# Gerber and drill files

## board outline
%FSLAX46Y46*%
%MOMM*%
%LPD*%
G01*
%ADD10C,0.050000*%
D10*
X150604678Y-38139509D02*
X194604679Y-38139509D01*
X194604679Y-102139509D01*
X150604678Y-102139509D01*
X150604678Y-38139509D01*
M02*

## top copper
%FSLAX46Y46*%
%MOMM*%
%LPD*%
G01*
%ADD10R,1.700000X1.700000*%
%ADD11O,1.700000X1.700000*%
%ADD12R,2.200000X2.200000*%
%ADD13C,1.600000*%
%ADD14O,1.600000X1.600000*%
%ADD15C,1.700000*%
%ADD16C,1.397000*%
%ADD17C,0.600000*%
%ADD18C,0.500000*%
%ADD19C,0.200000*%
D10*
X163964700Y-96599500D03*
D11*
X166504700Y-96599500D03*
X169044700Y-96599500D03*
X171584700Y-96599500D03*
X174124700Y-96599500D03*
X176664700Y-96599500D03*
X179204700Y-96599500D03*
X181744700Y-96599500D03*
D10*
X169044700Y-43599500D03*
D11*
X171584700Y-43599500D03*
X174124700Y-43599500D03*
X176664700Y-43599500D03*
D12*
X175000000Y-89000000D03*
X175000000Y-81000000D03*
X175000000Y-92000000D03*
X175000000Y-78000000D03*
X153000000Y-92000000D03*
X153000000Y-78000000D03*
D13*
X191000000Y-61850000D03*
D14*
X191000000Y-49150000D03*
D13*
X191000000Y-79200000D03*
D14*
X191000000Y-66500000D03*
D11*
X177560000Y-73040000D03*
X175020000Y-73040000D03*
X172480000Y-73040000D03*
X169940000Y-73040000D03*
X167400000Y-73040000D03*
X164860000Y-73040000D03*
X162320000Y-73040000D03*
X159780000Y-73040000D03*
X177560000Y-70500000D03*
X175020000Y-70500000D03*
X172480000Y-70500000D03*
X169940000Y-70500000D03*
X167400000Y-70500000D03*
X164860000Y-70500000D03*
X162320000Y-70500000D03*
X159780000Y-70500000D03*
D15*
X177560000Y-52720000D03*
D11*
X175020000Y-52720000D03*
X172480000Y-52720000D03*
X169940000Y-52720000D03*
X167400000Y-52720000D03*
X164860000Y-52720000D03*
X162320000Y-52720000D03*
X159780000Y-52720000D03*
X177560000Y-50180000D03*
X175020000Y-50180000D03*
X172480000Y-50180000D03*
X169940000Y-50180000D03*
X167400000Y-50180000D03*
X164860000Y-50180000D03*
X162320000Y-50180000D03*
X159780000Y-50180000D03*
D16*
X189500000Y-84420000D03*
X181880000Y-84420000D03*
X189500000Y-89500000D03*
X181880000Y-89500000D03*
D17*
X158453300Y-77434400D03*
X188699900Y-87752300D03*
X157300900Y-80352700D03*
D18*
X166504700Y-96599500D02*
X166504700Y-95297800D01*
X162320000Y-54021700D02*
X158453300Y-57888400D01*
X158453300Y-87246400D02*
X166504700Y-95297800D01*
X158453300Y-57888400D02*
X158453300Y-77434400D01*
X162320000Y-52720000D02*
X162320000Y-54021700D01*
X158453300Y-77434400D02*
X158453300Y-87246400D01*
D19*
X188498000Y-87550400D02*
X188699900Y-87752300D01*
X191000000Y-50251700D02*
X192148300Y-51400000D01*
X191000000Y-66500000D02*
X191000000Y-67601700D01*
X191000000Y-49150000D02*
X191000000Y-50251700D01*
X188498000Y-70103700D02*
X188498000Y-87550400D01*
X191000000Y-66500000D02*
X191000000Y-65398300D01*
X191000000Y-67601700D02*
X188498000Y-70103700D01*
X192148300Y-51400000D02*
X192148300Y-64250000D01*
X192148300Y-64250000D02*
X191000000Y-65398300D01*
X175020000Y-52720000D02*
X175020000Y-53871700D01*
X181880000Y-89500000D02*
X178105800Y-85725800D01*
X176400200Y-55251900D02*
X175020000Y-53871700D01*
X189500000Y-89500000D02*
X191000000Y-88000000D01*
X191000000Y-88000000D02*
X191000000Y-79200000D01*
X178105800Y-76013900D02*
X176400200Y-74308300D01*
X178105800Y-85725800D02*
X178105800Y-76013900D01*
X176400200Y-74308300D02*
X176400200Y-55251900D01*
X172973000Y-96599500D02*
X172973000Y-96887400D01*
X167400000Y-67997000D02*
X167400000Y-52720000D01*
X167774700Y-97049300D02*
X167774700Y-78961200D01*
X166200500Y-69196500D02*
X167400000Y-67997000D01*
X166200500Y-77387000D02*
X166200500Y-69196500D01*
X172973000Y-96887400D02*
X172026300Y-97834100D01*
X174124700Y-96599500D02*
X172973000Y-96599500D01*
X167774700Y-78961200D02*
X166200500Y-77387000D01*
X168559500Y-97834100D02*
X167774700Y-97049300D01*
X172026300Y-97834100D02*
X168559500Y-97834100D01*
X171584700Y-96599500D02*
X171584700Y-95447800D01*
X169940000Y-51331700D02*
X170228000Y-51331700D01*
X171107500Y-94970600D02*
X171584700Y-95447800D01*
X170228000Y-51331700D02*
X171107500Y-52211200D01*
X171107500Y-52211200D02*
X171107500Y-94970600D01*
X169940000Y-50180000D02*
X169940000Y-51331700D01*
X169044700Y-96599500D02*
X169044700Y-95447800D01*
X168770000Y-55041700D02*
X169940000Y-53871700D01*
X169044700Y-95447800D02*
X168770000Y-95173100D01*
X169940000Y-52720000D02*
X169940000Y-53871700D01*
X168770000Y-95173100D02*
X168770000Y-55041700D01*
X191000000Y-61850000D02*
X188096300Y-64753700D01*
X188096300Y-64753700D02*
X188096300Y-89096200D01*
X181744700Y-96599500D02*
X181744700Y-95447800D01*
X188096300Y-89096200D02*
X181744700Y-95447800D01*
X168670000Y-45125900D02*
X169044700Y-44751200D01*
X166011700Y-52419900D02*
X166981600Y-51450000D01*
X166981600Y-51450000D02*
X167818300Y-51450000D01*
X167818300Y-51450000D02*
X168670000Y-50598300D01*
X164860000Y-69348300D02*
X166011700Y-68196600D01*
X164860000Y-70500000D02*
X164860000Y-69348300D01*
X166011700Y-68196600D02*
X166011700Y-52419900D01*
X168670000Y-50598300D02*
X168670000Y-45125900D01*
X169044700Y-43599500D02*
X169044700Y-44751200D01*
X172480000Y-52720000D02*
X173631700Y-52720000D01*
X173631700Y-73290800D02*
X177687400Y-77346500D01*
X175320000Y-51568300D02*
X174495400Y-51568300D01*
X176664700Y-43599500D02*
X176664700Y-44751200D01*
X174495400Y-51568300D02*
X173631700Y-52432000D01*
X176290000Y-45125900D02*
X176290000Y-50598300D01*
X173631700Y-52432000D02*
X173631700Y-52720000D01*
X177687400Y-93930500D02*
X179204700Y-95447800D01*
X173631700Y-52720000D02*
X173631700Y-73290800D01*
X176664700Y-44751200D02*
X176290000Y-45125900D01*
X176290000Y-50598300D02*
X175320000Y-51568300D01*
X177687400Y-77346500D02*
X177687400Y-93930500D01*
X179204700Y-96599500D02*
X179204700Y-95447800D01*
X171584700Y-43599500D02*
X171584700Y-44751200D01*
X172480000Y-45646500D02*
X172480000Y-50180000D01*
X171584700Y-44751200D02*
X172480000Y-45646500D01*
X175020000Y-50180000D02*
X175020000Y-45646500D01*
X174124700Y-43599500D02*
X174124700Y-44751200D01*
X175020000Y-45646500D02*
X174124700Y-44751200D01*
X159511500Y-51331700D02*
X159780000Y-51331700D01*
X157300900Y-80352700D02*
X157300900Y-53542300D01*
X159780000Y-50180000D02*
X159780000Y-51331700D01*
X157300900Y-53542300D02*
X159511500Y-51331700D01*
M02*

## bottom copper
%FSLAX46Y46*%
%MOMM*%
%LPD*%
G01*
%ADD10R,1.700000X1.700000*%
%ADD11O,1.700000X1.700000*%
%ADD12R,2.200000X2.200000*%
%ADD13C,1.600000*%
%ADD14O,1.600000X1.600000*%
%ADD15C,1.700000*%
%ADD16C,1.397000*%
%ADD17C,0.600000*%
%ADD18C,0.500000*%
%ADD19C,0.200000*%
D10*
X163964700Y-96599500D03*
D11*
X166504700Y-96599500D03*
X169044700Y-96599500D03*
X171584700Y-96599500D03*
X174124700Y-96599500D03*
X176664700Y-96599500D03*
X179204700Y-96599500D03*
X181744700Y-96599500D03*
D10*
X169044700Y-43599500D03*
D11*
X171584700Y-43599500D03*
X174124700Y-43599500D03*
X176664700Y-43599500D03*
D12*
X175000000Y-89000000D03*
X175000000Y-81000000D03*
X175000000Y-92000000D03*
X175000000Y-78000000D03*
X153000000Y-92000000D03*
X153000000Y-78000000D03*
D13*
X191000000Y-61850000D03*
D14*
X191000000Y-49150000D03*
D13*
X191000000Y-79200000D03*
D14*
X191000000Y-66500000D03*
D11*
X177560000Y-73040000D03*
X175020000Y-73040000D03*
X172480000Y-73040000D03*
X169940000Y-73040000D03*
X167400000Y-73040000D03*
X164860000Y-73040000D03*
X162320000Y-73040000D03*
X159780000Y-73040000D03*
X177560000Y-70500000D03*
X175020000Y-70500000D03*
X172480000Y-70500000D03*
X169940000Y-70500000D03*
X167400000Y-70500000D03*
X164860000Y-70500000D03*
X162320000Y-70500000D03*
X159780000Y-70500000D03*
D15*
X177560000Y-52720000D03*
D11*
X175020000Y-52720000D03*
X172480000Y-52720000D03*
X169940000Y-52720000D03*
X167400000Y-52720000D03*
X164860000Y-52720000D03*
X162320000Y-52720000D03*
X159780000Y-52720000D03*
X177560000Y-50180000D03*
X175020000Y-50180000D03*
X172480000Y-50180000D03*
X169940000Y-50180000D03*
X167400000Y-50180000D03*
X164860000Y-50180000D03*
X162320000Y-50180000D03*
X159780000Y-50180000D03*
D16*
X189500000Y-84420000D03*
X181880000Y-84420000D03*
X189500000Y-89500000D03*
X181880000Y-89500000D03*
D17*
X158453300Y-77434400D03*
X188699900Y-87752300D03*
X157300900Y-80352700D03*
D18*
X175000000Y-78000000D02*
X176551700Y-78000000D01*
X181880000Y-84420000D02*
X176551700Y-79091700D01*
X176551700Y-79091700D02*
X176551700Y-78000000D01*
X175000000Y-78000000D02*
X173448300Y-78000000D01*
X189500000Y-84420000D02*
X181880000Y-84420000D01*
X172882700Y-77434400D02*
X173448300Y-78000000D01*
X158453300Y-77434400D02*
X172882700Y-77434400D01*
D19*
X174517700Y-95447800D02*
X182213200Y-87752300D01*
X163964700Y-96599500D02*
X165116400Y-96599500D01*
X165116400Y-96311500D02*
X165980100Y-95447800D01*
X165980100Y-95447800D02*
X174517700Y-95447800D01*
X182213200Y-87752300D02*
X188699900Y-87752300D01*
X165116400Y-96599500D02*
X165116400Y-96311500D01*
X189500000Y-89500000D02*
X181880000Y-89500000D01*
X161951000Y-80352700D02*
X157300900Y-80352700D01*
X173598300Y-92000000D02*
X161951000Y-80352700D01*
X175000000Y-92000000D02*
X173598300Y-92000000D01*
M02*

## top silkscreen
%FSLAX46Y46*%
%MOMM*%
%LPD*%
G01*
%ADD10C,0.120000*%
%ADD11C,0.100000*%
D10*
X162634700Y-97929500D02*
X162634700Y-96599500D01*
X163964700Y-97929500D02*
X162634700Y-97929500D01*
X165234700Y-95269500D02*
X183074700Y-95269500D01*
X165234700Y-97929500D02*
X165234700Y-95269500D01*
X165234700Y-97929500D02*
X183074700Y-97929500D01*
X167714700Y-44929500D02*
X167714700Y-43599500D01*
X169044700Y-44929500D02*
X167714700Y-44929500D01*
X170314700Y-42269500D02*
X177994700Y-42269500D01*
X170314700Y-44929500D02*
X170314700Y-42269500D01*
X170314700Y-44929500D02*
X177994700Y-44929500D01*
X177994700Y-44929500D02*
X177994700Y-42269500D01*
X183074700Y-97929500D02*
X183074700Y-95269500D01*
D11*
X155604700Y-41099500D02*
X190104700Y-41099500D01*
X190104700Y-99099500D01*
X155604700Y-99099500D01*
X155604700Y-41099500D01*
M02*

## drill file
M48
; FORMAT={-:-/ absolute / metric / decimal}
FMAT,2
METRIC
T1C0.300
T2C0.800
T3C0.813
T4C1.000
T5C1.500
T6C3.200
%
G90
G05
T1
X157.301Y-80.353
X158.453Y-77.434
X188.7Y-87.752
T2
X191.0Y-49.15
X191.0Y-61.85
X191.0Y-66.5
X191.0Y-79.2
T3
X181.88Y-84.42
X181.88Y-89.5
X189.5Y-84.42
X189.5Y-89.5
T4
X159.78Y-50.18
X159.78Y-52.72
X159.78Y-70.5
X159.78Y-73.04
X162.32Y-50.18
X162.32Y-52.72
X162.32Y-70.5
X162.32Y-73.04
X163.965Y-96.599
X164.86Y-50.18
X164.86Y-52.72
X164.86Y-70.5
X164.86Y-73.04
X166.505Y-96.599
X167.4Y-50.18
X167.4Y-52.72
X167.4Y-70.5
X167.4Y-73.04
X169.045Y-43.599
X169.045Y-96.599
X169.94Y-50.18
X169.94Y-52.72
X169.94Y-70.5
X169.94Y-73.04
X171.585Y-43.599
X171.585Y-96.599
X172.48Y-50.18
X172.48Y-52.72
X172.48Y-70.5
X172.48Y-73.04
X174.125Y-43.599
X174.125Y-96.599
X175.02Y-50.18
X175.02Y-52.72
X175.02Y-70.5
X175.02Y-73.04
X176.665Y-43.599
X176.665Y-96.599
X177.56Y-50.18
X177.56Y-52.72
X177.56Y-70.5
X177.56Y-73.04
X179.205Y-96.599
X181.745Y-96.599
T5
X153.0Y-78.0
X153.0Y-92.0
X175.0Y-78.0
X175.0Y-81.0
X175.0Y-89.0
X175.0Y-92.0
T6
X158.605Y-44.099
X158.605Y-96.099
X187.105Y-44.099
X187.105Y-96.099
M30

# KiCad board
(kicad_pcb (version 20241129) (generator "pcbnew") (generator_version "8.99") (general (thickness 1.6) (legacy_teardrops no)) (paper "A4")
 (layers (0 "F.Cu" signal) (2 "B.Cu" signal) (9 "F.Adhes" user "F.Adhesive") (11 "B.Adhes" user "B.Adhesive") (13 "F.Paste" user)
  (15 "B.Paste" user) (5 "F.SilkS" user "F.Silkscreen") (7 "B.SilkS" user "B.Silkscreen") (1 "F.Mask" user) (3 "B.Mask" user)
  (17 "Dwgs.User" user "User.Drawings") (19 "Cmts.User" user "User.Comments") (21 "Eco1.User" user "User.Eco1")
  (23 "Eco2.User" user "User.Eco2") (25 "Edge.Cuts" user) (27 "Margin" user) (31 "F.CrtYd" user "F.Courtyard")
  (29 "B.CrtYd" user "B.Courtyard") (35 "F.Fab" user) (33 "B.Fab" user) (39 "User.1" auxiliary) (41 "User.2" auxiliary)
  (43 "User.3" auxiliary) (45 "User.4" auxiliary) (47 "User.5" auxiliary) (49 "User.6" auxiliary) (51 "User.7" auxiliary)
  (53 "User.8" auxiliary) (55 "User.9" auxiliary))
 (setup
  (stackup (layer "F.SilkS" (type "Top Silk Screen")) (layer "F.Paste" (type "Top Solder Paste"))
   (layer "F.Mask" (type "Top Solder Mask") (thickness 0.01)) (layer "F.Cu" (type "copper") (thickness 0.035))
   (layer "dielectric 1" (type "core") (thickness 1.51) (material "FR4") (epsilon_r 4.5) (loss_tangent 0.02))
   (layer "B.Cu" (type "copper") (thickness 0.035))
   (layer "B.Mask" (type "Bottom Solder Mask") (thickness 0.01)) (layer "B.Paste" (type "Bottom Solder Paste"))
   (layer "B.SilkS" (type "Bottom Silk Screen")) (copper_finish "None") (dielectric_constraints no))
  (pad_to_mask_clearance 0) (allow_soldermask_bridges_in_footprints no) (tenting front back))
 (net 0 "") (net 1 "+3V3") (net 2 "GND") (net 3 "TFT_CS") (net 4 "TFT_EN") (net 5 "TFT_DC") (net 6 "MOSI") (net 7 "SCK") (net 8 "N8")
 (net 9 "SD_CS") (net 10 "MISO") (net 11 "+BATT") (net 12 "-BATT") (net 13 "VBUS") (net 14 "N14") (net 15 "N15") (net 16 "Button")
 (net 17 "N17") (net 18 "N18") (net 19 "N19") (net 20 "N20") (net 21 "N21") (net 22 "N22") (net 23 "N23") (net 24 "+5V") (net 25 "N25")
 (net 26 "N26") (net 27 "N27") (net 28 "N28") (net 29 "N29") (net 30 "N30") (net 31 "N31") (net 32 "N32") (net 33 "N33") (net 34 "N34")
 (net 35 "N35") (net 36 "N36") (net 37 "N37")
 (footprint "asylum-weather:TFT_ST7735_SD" (layer "F.Cu") (at 172.6047 76.5995 90)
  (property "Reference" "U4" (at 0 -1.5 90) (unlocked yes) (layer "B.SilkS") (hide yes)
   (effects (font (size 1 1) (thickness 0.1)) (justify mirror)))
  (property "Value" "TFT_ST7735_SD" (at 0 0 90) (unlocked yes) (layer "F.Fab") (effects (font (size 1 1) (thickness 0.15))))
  (fp_line (start -21.33 -9.97) (end -20 -9.97) (stroke (width 0.12) (type solid)) (layer "F.SilkS"))
  (fp_line (start -21.33 -8.64) (end -21.33 -9.97) (stroke (width 0.12) (type solid)) (layer "F.SilkS"))
  (fp_line (start -18.67 -7.37) (end -18.67 10.47) (stroke (width 0.12) (type solid)) (layer "F.SilkS"))
  (fp_line (start -21.33 -7.37) (end -18.67 -7.37) (stroke (width 0.12) (type solid)) (layer "F.SilkS"))
  (fp_line (start -21.33 -7.37) (end -21.33 10.47) (stroke (width 0.12) (type solid)) (layer "F.SilkS"))
  (fp_line (start 31.67 -4.89) (end 33 -4.89) (stroke (width 0.12) (type solid)) (layer "F.SilkS"))
  (fp_line (start 31.67 -3.56) (end 31.67 -4.89) (stroke (width 0.12) (type solid)) (layer "F.SilkS"))
  (fp_line (start 34.33 -2.29) (end 34.33 5.39) (stroke (width 0.12) (type solid)) (layer "F.SilkS"))
  (fp_line (start 31.67 -2.29) (end 34.33 -2.29) (stroke (width 0.12) (type solid)) (layer "F.SilkS"))
  (fp_line (start 31.67 -2.29) (end 31.67 5.39) (stroke (width 0.12) (type solid)) (layer "F.SilkS"))
  (fp_line (start 31.67 5.39) (end 34.33 5.39) (stroke (width 0.12) (type solid)) (layer "F.SilkS"))
  (fp_line (start -21.33 10.47) (end -18.67 10.47) (stroke (width 0.12) (type solid)) (layer "F.SilkS"))
  (fp_rect (start -22.5 -17) (end 35.5 17.5) (stroke (width 0.1) (type default)) (fill no) (layer "F.SilkS"))
  (pad "" np_thru_hole circle (at -19.5 -14 90) (size 3.2 3.2) (drill 3.2) (layers "*.Cu" "*.Mask"))
  (pad "" np_thru_hole circle (at -19.5 14.5 90) (size 3.2 3.2) (drill 3.2) (layers "*.Cu" "*.Mask"))
  (pad "" np_thru_hole circle (at 32.5 -14 90) (size 3.2 3.2) (drill 3.2) (layers "*.Cu" "*.Mask"))
  (pad "" np_thru_hole circle (at 32.5 14.5 90) (size 3.2 3.2) (drill 3.2) (layers "*.Cu" "*.Mask"))
  (pad "1" thru_hole rect (at -20 -8.64 90) (size 1.7 1.7) (drill 1) (layers "*.Cu" "*.Mask") (remove_unused_layers no) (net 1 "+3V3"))
  (pad "2" thru_hole oval (at -20 -6.1 90) (size 1.7 1.7) (drill 1) (layers "*.Cu" "*.Mask") (remove_unused_layers no) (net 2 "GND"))
  (pad "3" thru_hole oval (at -20 -3.56 90) (size 1.7 1.7) (drill 1) (layers "*.Cu" "*.Mask") (remove_unused_layers no) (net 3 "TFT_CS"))
  (pad "4" thru_hole oval (at -20 -1.02 90) (size 1.7 1.7) (drill 1) (layers "*.Cu" "*.Mask") (remove_unused_layers no) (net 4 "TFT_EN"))
  (pad "5" thru_hole oval (at -20 1.52 90) (size 1.7 1.7) (drill 1) (layers "*.Cu" "*.Mask") (remove_unused_layers no) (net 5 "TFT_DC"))
  (pad "6" thru_hole oval (at -20 4.06 90) (size 1.7 1.7) (drill 1) (layers "*.Cu" "*.Mask") (remove_unused_layers no) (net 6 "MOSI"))
  (pad "7" thru_hole oval (at -20 6.6 90) (size 1.7 1.7) (drill 1) (layers "*.Cu" "*.Mask") (remove_unused_layers no) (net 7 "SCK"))
  (pad "8" thru_hole oval (at -20 9.14 90) (size 1.7 1.7) (drill 1) (layers "*.Cu" "*.Mask") (remove_unused_layers no) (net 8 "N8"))
  (pad "9" thru_hole rect (at 33 -3.56 90) (size 1.7 1.7) (drill 1) (layers "*.Cu" "*.Mask") (remove_unused_layers no) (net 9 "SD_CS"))
  (pad "10" thru_hole oval (at 33 -1.02 90) (size 1.7 1.7) (drill 1) (layers "*.Cu" "*.Mask") (remove_unused_layers no) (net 6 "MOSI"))
  (pad "11" thru_hole oval (at 33 1.52 90) (size 1.7 1.7) (drill 1) (layers "*.Cu" "*.Mask") (remove_unused_layers no) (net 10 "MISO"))
  (pad "12" thru_hole oval (at 33 4.06 90) (size 1.7 1.7) (drill 1) (layers "*.Cu" "*.Mask") (remove_unused_layers no) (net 7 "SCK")))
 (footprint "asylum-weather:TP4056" (layer "B.Cu") (at 164.5 85 -90)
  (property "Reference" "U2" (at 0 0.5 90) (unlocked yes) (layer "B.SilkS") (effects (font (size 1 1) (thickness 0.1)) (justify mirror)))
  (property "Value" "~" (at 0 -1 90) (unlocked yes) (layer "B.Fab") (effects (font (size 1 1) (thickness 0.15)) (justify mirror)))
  (pad "0" thru_hole rect (at 4 -10.5 180) (size 2.2 2.2) (drill 1.5) (layers "F&B.Cu" "*.Mask") (remove_unused_layers no) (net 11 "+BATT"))
  (pad "1" thru_hole rect (at -4 -10.5 180) (size 2.2 2.2) (drill 1.5) (layers "F&B.Cu" "*.Mask") (remove_unused_layers no) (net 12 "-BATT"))
  (pad "2" thru_hole rect (at 7 -10.5 180) (size 2.2 2.2) (drill 1.5) (layers "F&B.Cu" "*.Mask") (remove_unused_layers no) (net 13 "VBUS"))
  (pad "3" thru_hole rect (at -7 -10.5 180) (size 2.2 2.2) (drill 1.5) (layers "F&B.Cu" "*.Mask") (remove_unused_layers no) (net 2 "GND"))
  (pad "4" thru_hole rect (at 7 11.5 180) (size 2.2 2.2) (drill 1.5) (layers "F&B.Cu" "*.Mask") (remove_unused_layers no) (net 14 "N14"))
  (pad "5" thru_hole rect (at -7 11.5 180) (size 2.2 2.2) (drill 1.5) (layers "F&B.Cu" "*.Mask") (remove_unused_layers no) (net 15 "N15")))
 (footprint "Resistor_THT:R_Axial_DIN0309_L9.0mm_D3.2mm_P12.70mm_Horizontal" (layer "B.Cu") (at 191 61.85 90)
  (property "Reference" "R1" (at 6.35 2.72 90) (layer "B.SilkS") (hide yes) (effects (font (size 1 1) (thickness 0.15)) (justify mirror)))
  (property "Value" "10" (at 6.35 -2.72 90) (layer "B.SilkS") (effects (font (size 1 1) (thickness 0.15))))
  (pad "1" thru_hole circle (at 0 0 90) (size 1.6 1.6) (drill 0.8) (layers "F&B.Cu" "*.Mask") (remove_unused_layers no) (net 8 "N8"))
  (pad "2" thru_hole oval (at 12.7 0 90) (size 1.6 1.6) (drill 0.8) (layers "F&B.Cu" "*.Mask") (remove_unused_layers no) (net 1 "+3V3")))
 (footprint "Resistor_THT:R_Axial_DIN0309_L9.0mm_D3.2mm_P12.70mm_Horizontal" (layer "B.Cu") (at 191 79.2 90)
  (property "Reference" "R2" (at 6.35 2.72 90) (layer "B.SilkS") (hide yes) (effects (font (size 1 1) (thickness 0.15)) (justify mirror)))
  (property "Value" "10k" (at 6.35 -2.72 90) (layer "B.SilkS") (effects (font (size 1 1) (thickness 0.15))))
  (pad "1" thru_hole circle (at 0 0 90) (size 1.6 1.6) (drill 0.8) (layers "F&B.Cu" "*.Mask") (remove_unused_layers no) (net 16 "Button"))
  (pad "2" thru_hole oval (at 12.7 0 90) (size 1.6 1.6) (drill 0.8) (layers "F&B.Cu" "*.Mask") (remove_unused_layers no) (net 1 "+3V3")))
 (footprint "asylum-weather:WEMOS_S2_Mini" (layer "B.Cu") (at 170.06 61.61 90)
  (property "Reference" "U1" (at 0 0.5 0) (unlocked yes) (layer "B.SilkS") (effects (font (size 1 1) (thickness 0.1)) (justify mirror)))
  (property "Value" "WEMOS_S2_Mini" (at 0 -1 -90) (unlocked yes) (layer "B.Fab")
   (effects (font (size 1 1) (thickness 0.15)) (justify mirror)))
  (pad "1" thru_hole oval (at -11.43 7.5 90) (size 1.7 1.7) (drill 1) (layers "F&B.Cu" "*.Mask") (remove_unused_layers no) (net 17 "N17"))
  (pad "2" thru_hole oval (at -11.43 4.96 90) (size 1.7 1.7) (drill 1) (layers "F&B.Cu" "*.Mask") (remove_unused_layers no) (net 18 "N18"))
  (pad "3" thru_hole oval (at -11.43 2.42 90) (size 1.7 1.7) (drill 1) (layers "F&B.Cu" "*.Mask") (remove_unused_layers no) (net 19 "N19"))
  (pad "4" thru_hole oval (at -11.43 -0.12 90) (size 1.7 1.7) (drill 1) (layers "F&B.Cu" "*.Mask") (remove_unused_layers no) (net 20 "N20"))
  (pad "5" thru_hole oval (at -11.43 -2.66 90) (size 1.7 1.7) (drill 1) (layers "F&B.Cu" "*.Mask") (remove_unused_layers no) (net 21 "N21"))
  (pad "6" thru_hole oval (at -11.43 -5.2 90) (size 1.7 1.7) (drill 1) (layers "F&B.Cu" "*.Mask") (remove_unused_layers no) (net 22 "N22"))
  (pad "7" thru_hole oval (at -11.43 -7.74 90) (size 1.7 1.7) (drill 1) (layers "F&B.Cu" "*.Mask") (remove_unused_layers no) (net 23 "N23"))
  (pad "8" thru_hole oval (at -11.43 -10.28 90) (size 1.7 1.7) (drill 1) (layers "F&B.Cu" "*.Mask") (remove_unused_layers no) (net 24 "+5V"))
  (pad "9" thru_hole oval (at -8.89 7.5 90) (size 1.7 1.7) (drill 1) (layers "F&B.Cu" "*.Mask") (remove_unused_layers no) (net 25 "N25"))
  (pad "10" thru_hole oval (at -8.89 4.96 90) (size 1.7 1.7) (drill 1) (layers "F&B.Cu" "*.Mask") (remove_unused_layers no) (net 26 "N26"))
  (pad "11" thru_hole oval (at -8.89 2.42 90) (size 1.7 1.7) (drill 1) (layers "F&B.Cu" "*.Mask") (remove_unused_layers no) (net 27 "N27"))
  (pad "12" thru_hole oval (at -8.89 -0.12 90) (size 1.7 1.7) (drill 1) (layers "F&B.Cu" "*.Mask") (remove_unused_layers no) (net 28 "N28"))
  (pad "13" thru_hole oval (at -8.89 -2.66 90) (size 1.7 1.7) (drill 1) (layers "F&B.Cu" "*.Mask") (remove_unused_layers no) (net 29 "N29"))
  (pad "14" thru_hole oval (at -8.89 -5.2 90) (size 1.7 1.7) (drill 1) (layers "F&B.Cu" "*.Mask") (remove_unused_layers no) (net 9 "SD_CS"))
  (pad "15" thru_hole oval (at -8.89 -7.74 90) (size 1.7 1.7) (drill 1) (layers "F&B.Cu" "*.Mask") (remove_unused_layers no) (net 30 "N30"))
  (pad "16" thru_hole oval (at -8.89 -10.28 90) (size 1.7 1.7) (drill 1) (layers "F&B.Cu" "*.Mask") (remove_unused_layers no) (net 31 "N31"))
  (pad "17" thru_hole circle (at 8.89 7.5 90) (size 1.7 1.7) (drill 1) (layers "F&B.Cu" "*.Mask") (remove_unused_layers no) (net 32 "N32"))
  (pad "18" thru_hole oval (at 8.89 4.96 90) (size 1.7 1.7) (drill 1) (layers "F&B.Cu" "*.Mask") (remove_unused_layers no) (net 16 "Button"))
  (pad "19" thru_hole oval (at 8.89 2.42 90) (size 1.7 1.7) (drill 1) (layers "F&B.Cu" "*.Mask") (remove_unused_layers no) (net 7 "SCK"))
  (pad "20" thru_hole oval (at 8.89 -0.12 90) (size 1.7 1.7) (drill 1) (layers "F&B.Cu" "*.Mask") (remove_unused_layers no) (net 3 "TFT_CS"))
  (pad "21" thru_hole oval (at 8.89 -2.66 90) (size 1.7 1.7) (drill 1) (layers "F&B.Cu" "*.Mask") (remove_unused_layers no) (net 5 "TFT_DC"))
  (pad "22" thru_hole oval (at 8.89 -5.2 90) (size 1.7 1.7) (drill 1) (layers "F&B.Cu" "*.Mask") (remove_unused_layers no) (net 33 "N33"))
  (pad "23" thru_hole oval (at 8.89 -7.74 90) (size 1.7 1.7) (drill 1) (layers "F&B.Cu" "*.Mask") (remove_unused_layers no) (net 2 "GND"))
  (pad "24" thru_hole oval (at 8.89 -10.28 90) (size 1.7 1.7) (drill 1) (layers "F&B.Cu" "*.Mask") (remove_unused_layers no) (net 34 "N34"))
  (pad "25" thru_hole oval (at 11.43 7.5 90) (size 1.7 1.7) (drill 1) (layers "F&B.Cu" "*.Mask") (remove_unused_layers no) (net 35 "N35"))
  (pad "26" thru_hole oval (at 11.43 4.96 90) (size 1.7 1.7) (drill 1) (layers "F&B.Cu" "*.Mask") (remove_unused_layers no) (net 10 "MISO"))
  (pad "27" thru_hole oval (at 11.43 2.42 90) (size 1.7 1.7) (drill 1) (layers "F&B.Cu" "*.Mask") (remove_unused_layers no) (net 6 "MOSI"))
  (pad "28" thru_hole oval (at 11.43 -0.12 90) (size 1.7 1.7) (drill 1) (layers "F&B.Cu" "*.Mask") (remove_unused_layers no)
   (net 4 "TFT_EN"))
  (pad "29" thru_hole oval (at 11.43 -2.66 90) (size 1.7 1.7) (drill 1) (layers "F&B.Cu" "*.Mask") (remove_unused_layers no) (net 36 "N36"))
  (pad "30" thru_hole oval (at 11.43 -5.2 90) (size 1.7 1.7) (drill 1) (layers "F&B.Cu" "*.Mask") (remove_unused_layers no) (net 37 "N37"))
  (pad "31" thru_hole oval (at 11.43 -7.74 90) (size 1.7 1.7) (drill 1) (layers "F&B.Cu" "*.Mask") (remove_unused_layers no))
  (pad "32" thru_hole oval (at 11.43 -10.28 90) (size 1.7 1.7) (drill 1) (layers "F&B.Cu" "*.Mask") (remove_unused_layers no)
   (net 13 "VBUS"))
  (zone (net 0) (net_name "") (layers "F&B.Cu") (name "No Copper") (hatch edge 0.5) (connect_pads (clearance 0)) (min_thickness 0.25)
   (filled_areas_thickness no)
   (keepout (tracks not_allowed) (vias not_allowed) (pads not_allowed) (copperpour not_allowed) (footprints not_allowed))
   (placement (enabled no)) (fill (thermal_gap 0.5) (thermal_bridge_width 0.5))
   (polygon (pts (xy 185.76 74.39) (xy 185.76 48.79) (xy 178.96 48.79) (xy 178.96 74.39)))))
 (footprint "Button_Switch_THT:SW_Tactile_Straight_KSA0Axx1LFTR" (layer "B.Cu") (at 189.5 84.42 180)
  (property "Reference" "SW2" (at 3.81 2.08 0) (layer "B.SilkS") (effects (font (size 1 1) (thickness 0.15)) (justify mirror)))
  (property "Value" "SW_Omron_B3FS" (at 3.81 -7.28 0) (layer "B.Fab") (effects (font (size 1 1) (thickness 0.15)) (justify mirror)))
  (pad "1" thru_hole circle (at 0 0 180) (size 1.397 1.397) (drill 0.8128) (layers "F&B.Cu" "*.Mask") (remove_unused_layers no)
   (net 2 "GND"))
  (pad "1" thru_hole circle (at 7.62 0 180) (size 1.397 1.397) (drill 0.8128) (layers "F&B.Cu" "*.Mask") (remove_unused_layers no)
   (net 2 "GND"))
  (pad "2" thru_hole circle (at 0 -5.08 180) (size 1.397 1.397) (drill 0.8128) (layers "F&B.Cu" "*.Mask") (remove_unused_layers no)
   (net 16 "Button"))
  (pad "2" thru_hole circle (at 7.62 -5.08 180) (size 1.397 1.397) (drill 0.8128) (layers "F&B.Cu" "*.Mask") (remove_unused_layers no)
   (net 16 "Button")))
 (gr_rect (start 150.604678 38.139509) (end 194.604679 102.139509) (stroke (width 0.05) (type default)) (fill no) (layer "Edge.Cuts"))
 (segment (start 166.5047 96.5995) (end 166.5047 95.2978) (width 0.5) (layer "F.Cu") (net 2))
 (segment (start 162.32 54.0217) (end 158.4533 57.8884) (width 0.5) (layer "F.Cu") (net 2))
 (segment (start 158.4533 87.2464) (end 166.5047 95.2978) (width 0.5) (layer "F.Cu") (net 2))
 (segment (start 158.4533 57.8884) (end 158.4533 77.4344) (width 0.5) (layer "F.Cu") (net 2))
 (segment (start 162.32 52.72) (end 162.32 54.0217) (width 0.5) (layer "F.Cu") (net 2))
 (segment (start 158.4533 77.4344) (end 158.4533 87.2464) (width 0.5) (layer "F.Cu") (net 2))
 (via (at 158.4533 77.4344) (size 0.6) (drill 0.3) (layers "F.Cu" "B.Cu") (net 2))
 (segment (start 175 78) (end 176.5517 78) (width 0.5) (layer "B.Cu") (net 2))
 (segment (start 181.88 84.42) (end 176.5517 79.0917) (width 0.5) (layer "B.Cu") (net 2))
 (segment (start 176.5517 79.0917) (end 176.5517 78) (width 0.5) (layer "B.Cu") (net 2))
 (segment (start 175 78) (end 173.4483 78) (width 0.5) (layer "B.Cu") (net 2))
 (segment (start 189.5 84.42) (end 181.88 84.42) (width 0.5) (layer "B.Cu") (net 2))
 (segment (start 172.8827 77.4344) (end 173.4483 78) (width 0.5) (layer "B.Cu") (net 2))
 (segment (start 158.4533 77.4344) (end 172.8827 77.4344) (width 0.5) (layer "B.Cu") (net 2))
 (segment (start 188.498 87.5504) (end 188.6999 87.7523) (width 0.2) (layer "F.Cu") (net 1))
 (segment (start 191 50.2517) (end 192.1483 51.4) (width 0.2) (layer "F.Cu") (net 1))
 (segment (start 191 66.5) (end 191 67.6017) (width 0.2) (layer "F.Cu") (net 1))
 (segment (start 191 49.15) (end 191 50.2517) (width 0.2) (layer "F.Cu") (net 1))
 (segment (start 188.498 70.1037) (end 188.498 87.5504) (width 0.2) (layer "F.Cu") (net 1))
 (segment (start 191 66.5) (end 191 65.3983) (width 0.2) (layer "F.Cu") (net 1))
 (segment (start 191 67.6017) (end 188.498 70.1037) (width 0.2) (layer "F.Cu") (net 1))
 (segment (start 192.1483 51.4) (end 192.1483 64.25) (width 0.2) (layer "F.Cu") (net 1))
 (segment (start 192.1483 64.25) (end 191 65.3983) (width 0.2) (layer "F.Cu") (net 1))
 (via (at 188.6999 87.7523) (size 0.6) (drill 0.3) (layers "F.Cu" "B.Cu") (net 1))
 (segment (start 174.5177 95.4478) (end 182.2132 87.7523) (width 0.2) (layer "B.Cu") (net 1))
 (segment (start 163.9647 96.5995) (end 165.1164 96.5995) (width 0.2) (layer "B.Cu") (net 1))
 (segment (start 165.1164 96.3115) (end 165.9801 95.4478) (width 0.2) (layer "B.Cu") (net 1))
 (segment (start 165.9801 95.4478) (end 174.5177 95.4478) (width 0.2) (layer "B.Cu") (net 1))
 (segment (start 182.2132 87.7523) (end 188.6999 87.7523) (width 0.2) (layer "B.Cu") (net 1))
 (segment (start 165.1164 96.5995) (end 165.1164 96.3115) (width 0.2) (layer "B.Cu") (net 1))
 (segment (start 175.02 52.72) (end 175.02 53.8717) (width 0.2) (layer "F.Cu") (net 16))
 (segment (start 181.88 89.5) (end 178.1058 85.7258) (width 0.2) (layer "F.Cu") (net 16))
 (segment (start 176.4002 55.2519) (end 175.02 53.8717) (width 0.2) (layer "F.Cu") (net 16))
 (segment (start 189.5 89.5) (end 191 88) (width 0.2) (layer "F.Cu") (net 16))
 (segment (start 191 88) (end 191 79.2) (width 0.2) (layer "F.Cu") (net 16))
 (segment (start 178.1058 76.0139) (end 176.4002 74.3083) (width 0.2) (layer "F.Cu") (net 16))
 (segment (start 178.1058 85.7258) (end 178.1058 76.0139) (width 0.2) (layer "F.Cu") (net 16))
 (segment (start 176.4002 74.3083) (end 176.4002 55.2519) (width 0.2) (layer "F.Cu") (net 16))
 (segment (start 189.5 89.5) (end 181.88 89.5) (width 0.2) (layer "B.Cu") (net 16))
 (segment (start 172.973 96.5995) (end 172.973 96.8874) (width 0.2) (layer "F.Cu") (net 5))
 (segment (start 167.4 67.997) (end 167.4 52.72) (width 0.2) (layer "F.Cu") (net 5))
 (segment (start 167.7747 97.0493) (end 167.7747 78.9612) (width 0.2) (layer "F.Cu") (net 5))
 (segment (start 166.2005 69.1965) (end 167.4 67.997) (width 0.2) (layer "F.Cu") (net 5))
 (segment (start 166.2005 77.387) (end 166.2005 69.1965) (width 0.2) (layer "F.Cu") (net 5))
 (segment (start 172.973 96.8874) (end 172.0263 97.8341) (width 0.2) (layer "F.Cu") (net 5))
 (segment (start 174.1247 96.5995) (end 172.973 96.5995) (width 0.2) (layer "F.Cu") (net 5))
 (segment (start 167.7747 78.9612) (end 166.2005 77.387) (width 0.2) (layer "F.Cu") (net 5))
 (segment (start 168.5595 97.8341) (end 167.7747 97.0493) (width 0.2) (layer "F.Cu") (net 5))
 (segment (start 172.0263 97.8341) (end 168.5595 97.8341) (width 0.2) (layer "F.Cu") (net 5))
 (segment (start 171.5847 96.5995) (end 171.5847 95.4478) (width 0.2) (layer "F.Cu") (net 4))
 (segment (start 169.94 51.3317) (end 170.228 51.3317) (width 0.2) (layer "F.Cu") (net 4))
 (segment (start 171.1075 94.9706) (end 171.5847 95.4478) (width 0.2) (layer "F.Cu") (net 4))
 (segment (start 170.228 51.3317) (end 171.1075 52.2112) (width 0.2) (layer "F.Cu") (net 4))
 (segment (start 171.1075 52.2112) (end 171.1075 94.9706) (width 0.2) (layer "F.Cu") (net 4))
 (segment (start 169.94 50.18) (end 169.94 51.3317) (width 0.2) (layer "F.Cu") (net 4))
 (segment (start 169.0447 96.5995) (end 169.0447 95.4478) (width 0.2) (layer "F.Cu") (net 3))
 (segment (start 168.77 55.0417) (end 169.94 53.8717) (width 0.2) (layer "F.Cu") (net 3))
 (segment (start 169.0447 95.4478) (end 168.77 95.1731) (width 0.2) (layer "F.Cu") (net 3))
 (segment (start 169.94 52.72) (end 169.94 53.8717) (width 0.2) (layer "F.Cu") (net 3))
 (segment (start 168.77 95.1731) (end 168.77 55.0417) (width 0.2) (layer "F.Cu") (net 3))
 (segment (start 191 61.85) (end 188.0963 64.7537) (width 0.2) (layer "F.Cu") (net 8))
 (segment (start 188.0963 64.7537) (end 188.0963 89.0962) (width 0.2) (layer "F.Cu") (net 8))
 (segment (start 181.7447 96.5995) (end 181.7447 95.4478) (width 0.2) (layer "F.Cu") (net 8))
 (segment (start 188.0963 89.0962) (end 181.7447 95.4478) (width 0.2) (layer "F.Cu") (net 8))
 (segment (start 168.67 45.1259) (end 169.0447 44.7512) (width 0.2) (layer "F.Cu") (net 9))
 (segment (start 166.0117 52.4199) (end 166.9816 51.45) (width 0.2) (layer "F.Cu") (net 9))
 (segment (start 166.9816 51.45) (end 167.8183 51.45) (width 0.2) (layer "F.Cu") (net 9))
 (segment (start 167.8183 51.45) (end 168.67 50.5983) (width 0.2) (layer "F.Cu") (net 9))
 (segment (start 164.86 69.3483) (end 166.0117 68.1966) (width 0.2) (layer "F.Cu") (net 9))
 (segment (start 164.86 70.5) (end 164.86 69.3483) (width 0.2) (layer "F.Cu") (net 9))
 (segment (start 166.0117 68.1966) (end 166.0117 52.4199) (width 0.2) (layer "F.Cu") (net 9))
 (segment (start 168.67 50.5983) (end 168.67 45.1259) (width 0.2) (layer "F.Cu") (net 9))
 (segment (start 169.0447 43.5995) (end 169.0447 44.7512) (width 0.2) (layer "F.Cu") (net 9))
 (segment (start 172.48 52.72) (end 173.6317 52.72) (width 0.2) (layer "F.Cu") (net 7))
 (segment (start 173.6317 73.2908) (end 177.6874 77.3465) (width 0.2) (layer "F.Cu") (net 7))
 (segment (start 175.32 51.5683) (end 174.4954 51.5683) (width 0.2) (layer "F.Cu") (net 7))
 (segment (start 176.6647 43.5995) (end 176.6647 44.7512) (width 0.2) (layer "F.Cu") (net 7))
 (segment (start 174.4954 51.5683) (end 173.6317 52.432) (width 0.2) (layer "F.Cu") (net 7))
 (segment (start 176.29 45.1259) (end 176.29 50.5983) (width 0.2) (layer "F.Cu") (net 7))
 (segment (start 173.6317 52.432) (end 173.6317 52.72) (width 0.2) (layer "F.Cu") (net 7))
 (segment (start 177.6874 93.9305) (end 179.2047 95.4478) (width 0.2) (layer "F.Cu") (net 7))
 (segment (start 173.6317 52.72) (end 173.6317 73.2908) (width 0.2) (layer "F.Cu") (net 7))
 (segment (start 176.6647 44.7512) (end 176.29 45.1259) (width 0.2) (layer "F.Cu") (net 7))
 (segment (start 176.29 50.5983) (end 175.32 51.5683) (width 0.2) (layer "F.Cu") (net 7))
 (segment (start 177.6874 77.3465) (end 177.6874 93.9305) (width 0.2) (layer "F.Cu") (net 7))
 (segment (start 179.2047 96.5995) (end 179.2047 95.4478) (width 0.2) (layer "F.Cu") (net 7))
 (segment (start 171.5847 43.5995) (end 171.5847 44.7512) (width 0.2) (layer "F.Cu") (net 6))
 (segment (start 172.48 45.6465) (end 172.48 50.18) (width 0.2) (layer "F.Cu") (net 6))
 (segment (start 171.5847 44.7512) (end 172.48 45.6465) (width 0.2) (layer "F.Cu") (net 6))
 (segment (start 175.02 50.18) (end 175.02 45.6465) (width 0.2) (layer "F.Cu") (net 10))
 (segment (start 174.1247 43.5995) (end 174.1247 44.7512) (width 0.2) (layer "F.Cu") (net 10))
 (segment (start 175.02 45.6465) (end 174.1247 44.7512) (width 0.2) (layer "F.Cu") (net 10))
 (segment (start 159.5115 51.3317) (end 159.78 51.3317) (width 0.2) (layer "F.Cu") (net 13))
 (segment (start 157.3009 80.3527) (end 157.3009 53.5423) (width 0.2) (layer "F.Cu") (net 13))
 (segment (start 159.78 50.18) (end 159.78 51.3317) (width 0.2) (layer "F.Cu") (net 13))
 (segment (start 157.3009 53.5423) (end 159.5115 51.3317) (width 0.2) (layer "F.Cu") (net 13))
 (via (at 157.3009 80.3527) (size 0.6) (drill 0.3) (layers "F.Cu" "B.Cu") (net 13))
 (segment (start 161.951 80.3527) (end 157.3009 80.3527) (width 0.2) (layer "B.Cu") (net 13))
 (segment (start 173.5983 92) (end 161.951 80.3527) (width 0.2) (layer "B.Cu") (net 13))
 (segment (start 175 92) (end 173.5983 92) (width 0.2) (layer "B.Cu") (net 13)))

